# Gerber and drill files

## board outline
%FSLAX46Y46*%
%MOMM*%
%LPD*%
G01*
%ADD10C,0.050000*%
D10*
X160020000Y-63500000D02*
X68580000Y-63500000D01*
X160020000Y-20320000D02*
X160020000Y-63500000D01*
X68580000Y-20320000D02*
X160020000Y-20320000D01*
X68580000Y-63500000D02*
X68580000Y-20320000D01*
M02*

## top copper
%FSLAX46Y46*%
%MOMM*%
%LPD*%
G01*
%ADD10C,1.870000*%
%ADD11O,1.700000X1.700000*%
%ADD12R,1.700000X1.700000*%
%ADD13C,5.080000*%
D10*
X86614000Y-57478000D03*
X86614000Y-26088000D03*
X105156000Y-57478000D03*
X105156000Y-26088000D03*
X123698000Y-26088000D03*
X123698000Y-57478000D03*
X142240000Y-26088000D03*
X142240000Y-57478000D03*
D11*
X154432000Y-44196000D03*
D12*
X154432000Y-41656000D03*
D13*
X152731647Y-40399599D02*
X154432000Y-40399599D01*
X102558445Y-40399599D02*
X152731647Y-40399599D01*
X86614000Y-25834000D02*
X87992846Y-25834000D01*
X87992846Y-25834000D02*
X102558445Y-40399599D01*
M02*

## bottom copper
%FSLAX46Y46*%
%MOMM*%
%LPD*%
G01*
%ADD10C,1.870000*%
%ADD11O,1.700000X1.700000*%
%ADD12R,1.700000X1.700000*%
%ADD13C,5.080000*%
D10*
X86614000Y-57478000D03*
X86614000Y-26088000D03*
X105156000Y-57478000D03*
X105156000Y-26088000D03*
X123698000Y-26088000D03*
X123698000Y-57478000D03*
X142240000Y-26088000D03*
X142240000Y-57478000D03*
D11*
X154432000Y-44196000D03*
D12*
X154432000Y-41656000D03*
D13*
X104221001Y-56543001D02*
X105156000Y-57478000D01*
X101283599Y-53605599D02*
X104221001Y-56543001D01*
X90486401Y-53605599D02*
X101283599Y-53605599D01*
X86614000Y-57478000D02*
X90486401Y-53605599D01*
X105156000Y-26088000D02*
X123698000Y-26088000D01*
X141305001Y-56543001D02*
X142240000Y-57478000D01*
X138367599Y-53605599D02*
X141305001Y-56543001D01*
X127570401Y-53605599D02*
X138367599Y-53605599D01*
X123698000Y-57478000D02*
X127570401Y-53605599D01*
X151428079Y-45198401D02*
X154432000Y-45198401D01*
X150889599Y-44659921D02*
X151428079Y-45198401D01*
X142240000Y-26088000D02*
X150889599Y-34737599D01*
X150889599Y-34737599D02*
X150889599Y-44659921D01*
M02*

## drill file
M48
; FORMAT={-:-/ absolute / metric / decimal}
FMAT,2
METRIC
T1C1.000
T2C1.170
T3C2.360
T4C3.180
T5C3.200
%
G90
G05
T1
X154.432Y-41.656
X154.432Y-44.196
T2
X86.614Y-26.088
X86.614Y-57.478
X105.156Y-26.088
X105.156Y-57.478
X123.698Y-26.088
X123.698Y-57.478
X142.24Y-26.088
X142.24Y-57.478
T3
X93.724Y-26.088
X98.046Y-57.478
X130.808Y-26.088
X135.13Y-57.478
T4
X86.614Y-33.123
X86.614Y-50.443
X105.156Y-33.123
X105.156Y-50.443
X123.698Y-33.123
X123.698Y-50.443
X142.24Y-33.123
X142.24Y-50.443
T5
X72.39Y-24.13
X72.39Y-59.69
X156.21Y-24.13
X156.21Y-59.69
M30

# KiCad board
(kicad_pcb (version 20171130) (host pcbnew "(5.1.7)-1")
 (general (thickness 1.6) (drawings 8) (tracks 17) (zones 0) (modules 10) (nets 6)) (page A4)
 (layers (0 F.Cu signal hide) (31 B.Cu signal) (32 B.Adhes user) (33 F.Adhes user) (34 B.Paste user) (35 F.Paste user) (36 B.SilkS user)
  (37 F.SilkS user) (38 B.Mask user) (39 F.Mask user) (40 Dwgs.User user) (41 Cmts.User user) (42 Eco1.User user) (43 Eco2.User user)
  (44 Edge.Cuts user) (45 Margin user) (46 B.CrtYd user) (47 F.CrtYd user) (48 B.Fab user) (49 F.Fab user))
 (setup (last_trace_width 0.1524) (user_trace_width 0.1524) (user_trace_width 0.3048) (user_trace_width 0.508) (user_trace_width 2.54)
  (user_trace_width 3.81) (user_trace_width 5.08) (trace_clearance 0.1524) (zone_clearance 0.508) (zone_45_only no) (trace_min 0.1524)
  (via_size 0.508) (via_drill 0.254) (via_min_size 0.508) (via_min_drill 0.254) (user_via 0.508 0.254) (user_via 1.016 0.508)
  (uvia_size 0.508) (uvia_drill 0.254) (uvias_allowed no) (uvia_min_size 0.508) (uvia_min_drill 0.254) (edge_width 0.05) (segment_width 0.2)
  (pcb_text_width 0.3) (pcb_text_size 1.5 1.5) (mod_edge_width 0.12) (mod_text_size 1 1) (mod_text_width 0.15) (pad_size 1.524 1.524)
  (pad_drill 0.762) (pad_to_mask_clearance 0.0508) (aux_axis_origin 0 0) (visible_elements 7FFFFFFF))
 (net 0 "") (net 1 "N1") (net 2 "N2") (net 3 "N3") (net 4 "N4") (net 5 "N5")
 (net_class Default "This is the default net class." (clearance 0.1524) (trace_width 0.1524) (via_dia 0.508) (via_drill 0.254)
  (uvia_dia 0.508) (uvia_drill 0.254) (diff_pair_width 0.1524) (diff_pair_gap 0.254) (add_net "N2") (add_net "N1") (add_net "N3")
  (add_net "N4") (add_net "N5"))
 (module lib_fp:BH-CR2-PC (layer F.Cu) (at 86.614 41.783 90)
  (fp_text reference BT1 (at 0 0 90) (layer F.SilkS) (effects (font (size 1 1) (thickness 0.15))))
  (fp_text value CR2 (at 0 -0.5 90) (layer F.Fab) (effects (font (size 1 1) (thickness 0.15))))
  (pad 2 thru_hole circle (at -15.695 0 90) (size 1.87 1.87) (drill 1.17) (layers *.Cu *.Mask) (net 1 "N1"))
  (pad 1 thru_hole circle (at 15.695 0 90) (size 1.87 1.87) (drill 1.17) (layers *.Cu *.Mask) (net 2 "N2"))
  (pad "" np_thru_hole circle (at -8.66 0 90) (size 3.18 3.18) (drill 3.18) (layers *.Cu *.Mask))
  (pad "" np_thru_hole circle (at 8.66 0 90) (size 3.18 3.18) (drill 3.18) (layers *.Cu *.Mask))
  (pad "" np_thru_hole circle (at 15.695 7.11 90) (size 2.36 2.36) (drill 2.36) (layers *.Cu *.Mask)))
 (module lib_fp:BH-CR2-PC (layer F.Cu) (at 105.156 41.783 270)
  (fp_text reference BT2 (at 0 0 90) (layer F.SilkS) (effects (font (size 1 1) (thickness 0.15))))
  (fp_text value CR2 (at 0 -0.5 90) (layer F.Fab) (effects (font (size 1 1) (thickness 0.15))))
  (pad "" np_thru_hole circle (at 15.695 7.11 270) (size 2.36 2.36) (drill 2.36) (layers *.Cu *.Mask))
  (pad "" np_thru_hole circle (at 8.66 0 270) (size 3.18 3.18) (drill 3.18) (layers *.Cu *.Mask))
  (pad "" np_thru_hole circle (at -8.66 0 270) (size 3.18 3.18) (drill 3.18) (layers *.Cu *.Mask))
  (pad 1 thru_hole circle (at 15.695 0 270) (size 1.87 1.87) (drill 1.17) (layers *.Cu *.Mask) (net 1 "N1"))
  (pad 2 thru_hole circle (at -15.695 0 270) (size 1.87 1.87) (drill 1.17) (layers *.Cu *.Mask) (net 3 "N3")))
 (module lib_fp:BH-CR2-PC (layer F.Cu) (at 123.698 41.783 90)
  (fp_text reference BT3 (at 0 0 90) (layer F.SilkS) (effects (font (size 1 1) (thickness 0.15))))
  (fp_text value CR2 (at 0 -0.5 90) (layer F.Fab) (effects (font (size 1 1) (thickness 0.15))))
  (pad "" np_thru_hole circle (at 15.695 7.11 90) (size 2.36 2.36) (drill 2.36) (layers *.Cu *.Mask))
  (pad "" np_thru_hole circle (at 8.66 0 90) (size 3.18 3.18) (drill 3.18) (layers *.Cu *.Mask))
  (pad "" np_thru_hole circle (at -8.66 0 90) (size 3.18 3.18) (drill 3.18) (layers *.Cu *.Mask))
  (pad 1 thru_hole circle (at 15.695 0 90) (size 1.87 1.87) (drill 1.17) (layers *.Cu *.Mask) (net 3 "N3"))
  (pad 2 thru_hole circle (at -15.695 0 90) (size 1.87 1.87) (drill 1.17) (layers *.Cu *.Mask) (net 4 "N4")))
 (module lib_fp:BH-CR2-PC (layer F.Cu) (at 142.24 41.783 270)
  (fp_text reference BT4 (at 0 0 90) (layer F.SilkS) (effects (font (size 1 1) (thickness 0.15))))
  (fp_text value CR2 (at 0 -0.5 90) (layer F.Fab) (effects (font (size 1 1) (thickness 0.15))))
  (pad 2 thru_hole circle (at -15.695 0 270) (size 1.87 1.87) (drill 1.17) (layers *.Cu *.Mask) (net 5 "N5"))
  (pad 1 thru_hole circle (at 15.695 0 270) (size 1.87 1.87) (drill 1.17) (layers *.Cu *.Mask) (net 4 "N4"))
  (pad "" np_thru_hole circle (at -8.66 0 270) (size 3.18 3.18) (drill 3.18) (layers *.Cu *.Mask))
  (pad "" np_thru_hole circle (at 8.66 0 270) (size 3.18 3.18) (drill 3.18) (layers *.Cu *.Mask))
  (pad "" np_thru_hole circle (at 15.695 7.11 270) (size 2.36 2.36) (drill 2.36) (layers *.Cu *.Mask)))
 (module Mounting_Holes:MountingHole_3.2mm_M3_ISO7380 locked (layer F.Cu) (at 72.39 24.13)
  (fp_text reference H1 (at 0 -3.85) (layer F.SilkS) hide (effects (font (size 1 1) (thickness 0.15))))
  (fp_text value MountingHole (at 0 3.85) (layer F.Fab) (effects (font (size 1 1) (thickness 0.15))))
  (pad 1 np_thru_hole circle (at 0 0) (size 3.2 3.2) (drill 3.2) (layers *.Cu *.Mask)))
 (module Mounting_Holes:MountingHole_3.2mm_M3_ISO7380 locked (layer F.Cu) (at 72.39 59.69)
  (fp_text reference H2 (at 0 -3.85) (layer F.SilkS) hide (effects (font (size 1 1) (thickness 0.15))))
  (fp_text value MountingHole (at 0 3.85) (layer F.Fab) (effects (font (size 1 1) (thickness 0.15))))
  (pad 1 np_thru_hole circle (at 0 0) (size 3.2 3.2) (drill 3.2) (layers *.Cu *.Mask)))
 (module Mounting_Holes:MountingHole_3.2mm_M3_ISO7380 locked (layer F.Cu) (at 156.21 24.13)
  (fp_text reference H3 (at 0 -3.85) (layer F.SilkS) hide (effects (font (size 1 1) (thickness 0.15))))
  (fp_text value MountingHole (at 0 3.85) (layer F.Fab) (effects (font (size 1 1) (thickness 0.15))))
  (pad 1 np_thru_hole circle (at 0 0) (size 3.2 3.2) (drill 3.2) (layers *.Cu *.Mask)))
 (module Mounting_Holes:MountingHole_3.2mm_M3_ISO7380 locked (layer F.Cu) (at 156.21 59.69)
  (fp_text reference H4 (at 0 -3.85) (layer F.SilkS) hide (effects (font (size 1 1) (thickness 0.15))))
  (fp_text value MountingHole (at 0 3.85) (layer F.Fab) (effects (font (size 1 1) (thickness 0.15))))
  (pad 1 np_thru_hole circle (at 0 0) (size 3.2 3.2) (drill 3.2) (layers *.Cu *.Mask)))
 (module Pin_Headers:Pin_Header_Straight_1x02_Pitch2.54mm (layer F.Cu) (at 154.432 41.656)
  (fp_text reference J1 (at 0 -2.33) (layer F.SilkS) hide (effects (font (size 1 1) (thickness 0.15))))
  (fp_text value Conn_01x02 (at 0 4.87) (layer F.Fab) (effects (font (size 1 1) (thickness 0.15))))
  (pad 2 thru_hole oval (at 0 2.54) (size 1.7 1.7) (drill 1) (layers *.Cu *.Mask) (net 5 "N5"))
  (pad 1 thru_hole rect (at 0 0) (size 1.7 1.7) (drill 1) (layers *.Cu *.Mask) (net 2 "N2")))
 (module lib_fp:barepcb (layer F.Cu) (at 72.136 16.51)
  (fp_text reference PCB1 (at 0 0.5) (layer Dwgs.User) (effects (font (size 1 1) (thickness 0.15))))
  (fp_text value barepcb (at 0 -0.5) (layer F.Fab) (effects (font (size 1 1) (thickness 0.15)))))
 (gr_line (start 160.02 63.5) (end 68.58 63.5) (layer Edge.Cuts) (width 0.05))
 (gr_line (start 160.02 20.32) (end 160.02 63.5) (layer Edge.Cuts) (width 0.05))
 (gr_line (start 68.58 20.32) (end 160.02 20.32) (layer Edge.Cuts) (width 0.05))
 (gr_line (start 68.58 63.5) (end 68.58 20.32) (layer Edge.Cuts) (width 0.05))
 (segment (start 104.221001 56.543001) (end 105.156 57.478) (width 5.08) (layer B.Cu) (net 1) (status 20))
 (segment (start 101.283599 53.605599) (end 104.221001 56.543001) (width 5.08) (layer B.Cu) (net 1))
 (segment (start 90.486401 53.605599) (end 101.283599 53.605599) (width 5.08) (layer B.Cu) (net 1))
 (segment (start 86.614 57.478) (end 90.486401 53.605599) (width 5.08) (layer B.Cu) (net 1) (status 10))
 (segment (start 152.731647 40.399599) (end 154.432 40.399599) (width 5.08) (layer F.Cu) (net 2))
 (segment (start 102.558445 40.399599) (end 152.731647 40.399599) (width 5.08) (layer F.Cu) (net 2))
 (segment (start 86.614 25.834) (end 87.992846 25.834) (width 5.08) (layer F.Cu) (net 2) (status 10))
 (segment (start 87.992846 25.834) (end 102.558445 40.399599) (width 5.08) (layer F.Cu) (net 2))
 (segment (start 105.156 26.088) (end 123.698 26.088) (width 5.08) (layer B.Cu) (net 3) (status 30))
 (segment (start 141.305001 56.543001) (end 142.24 57.478) (width 5.08) (layer B.Cu) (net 4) (status 20))
 (segment (start 138.367599 53.605599) (end 141.305001 56.543001) (width 5.08) (layer B.Cu) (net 4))
 (segment (start 127.570401 53.605599) (end 138.367599 53.605599) (width 5.08) (layer B.Cu) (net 4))
 (segment (start 123.698 57.478) (end 127.570401 53.605599) (width 5.08) (layer B.Cu) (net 4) (status 10))
 (segment (start 151.428079 45.198401) (end 154.432 45.198401) (width 5.08) (layer B.Cu) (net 5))
 (segment (start 150.889599 44.659921) (end 151.428079 45.198401) (width 5.08) (layer B.Cu) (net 5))
 (segment (start 142.24 26.088) (end 150.889599 34.737599) (width 5.08) (layer B.Cu) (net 5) (status 10))
 (segment (start 150.889599 34.737599) (end 150.889599 44.659921) (width 5.08) (layer B.Cu) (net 5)))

